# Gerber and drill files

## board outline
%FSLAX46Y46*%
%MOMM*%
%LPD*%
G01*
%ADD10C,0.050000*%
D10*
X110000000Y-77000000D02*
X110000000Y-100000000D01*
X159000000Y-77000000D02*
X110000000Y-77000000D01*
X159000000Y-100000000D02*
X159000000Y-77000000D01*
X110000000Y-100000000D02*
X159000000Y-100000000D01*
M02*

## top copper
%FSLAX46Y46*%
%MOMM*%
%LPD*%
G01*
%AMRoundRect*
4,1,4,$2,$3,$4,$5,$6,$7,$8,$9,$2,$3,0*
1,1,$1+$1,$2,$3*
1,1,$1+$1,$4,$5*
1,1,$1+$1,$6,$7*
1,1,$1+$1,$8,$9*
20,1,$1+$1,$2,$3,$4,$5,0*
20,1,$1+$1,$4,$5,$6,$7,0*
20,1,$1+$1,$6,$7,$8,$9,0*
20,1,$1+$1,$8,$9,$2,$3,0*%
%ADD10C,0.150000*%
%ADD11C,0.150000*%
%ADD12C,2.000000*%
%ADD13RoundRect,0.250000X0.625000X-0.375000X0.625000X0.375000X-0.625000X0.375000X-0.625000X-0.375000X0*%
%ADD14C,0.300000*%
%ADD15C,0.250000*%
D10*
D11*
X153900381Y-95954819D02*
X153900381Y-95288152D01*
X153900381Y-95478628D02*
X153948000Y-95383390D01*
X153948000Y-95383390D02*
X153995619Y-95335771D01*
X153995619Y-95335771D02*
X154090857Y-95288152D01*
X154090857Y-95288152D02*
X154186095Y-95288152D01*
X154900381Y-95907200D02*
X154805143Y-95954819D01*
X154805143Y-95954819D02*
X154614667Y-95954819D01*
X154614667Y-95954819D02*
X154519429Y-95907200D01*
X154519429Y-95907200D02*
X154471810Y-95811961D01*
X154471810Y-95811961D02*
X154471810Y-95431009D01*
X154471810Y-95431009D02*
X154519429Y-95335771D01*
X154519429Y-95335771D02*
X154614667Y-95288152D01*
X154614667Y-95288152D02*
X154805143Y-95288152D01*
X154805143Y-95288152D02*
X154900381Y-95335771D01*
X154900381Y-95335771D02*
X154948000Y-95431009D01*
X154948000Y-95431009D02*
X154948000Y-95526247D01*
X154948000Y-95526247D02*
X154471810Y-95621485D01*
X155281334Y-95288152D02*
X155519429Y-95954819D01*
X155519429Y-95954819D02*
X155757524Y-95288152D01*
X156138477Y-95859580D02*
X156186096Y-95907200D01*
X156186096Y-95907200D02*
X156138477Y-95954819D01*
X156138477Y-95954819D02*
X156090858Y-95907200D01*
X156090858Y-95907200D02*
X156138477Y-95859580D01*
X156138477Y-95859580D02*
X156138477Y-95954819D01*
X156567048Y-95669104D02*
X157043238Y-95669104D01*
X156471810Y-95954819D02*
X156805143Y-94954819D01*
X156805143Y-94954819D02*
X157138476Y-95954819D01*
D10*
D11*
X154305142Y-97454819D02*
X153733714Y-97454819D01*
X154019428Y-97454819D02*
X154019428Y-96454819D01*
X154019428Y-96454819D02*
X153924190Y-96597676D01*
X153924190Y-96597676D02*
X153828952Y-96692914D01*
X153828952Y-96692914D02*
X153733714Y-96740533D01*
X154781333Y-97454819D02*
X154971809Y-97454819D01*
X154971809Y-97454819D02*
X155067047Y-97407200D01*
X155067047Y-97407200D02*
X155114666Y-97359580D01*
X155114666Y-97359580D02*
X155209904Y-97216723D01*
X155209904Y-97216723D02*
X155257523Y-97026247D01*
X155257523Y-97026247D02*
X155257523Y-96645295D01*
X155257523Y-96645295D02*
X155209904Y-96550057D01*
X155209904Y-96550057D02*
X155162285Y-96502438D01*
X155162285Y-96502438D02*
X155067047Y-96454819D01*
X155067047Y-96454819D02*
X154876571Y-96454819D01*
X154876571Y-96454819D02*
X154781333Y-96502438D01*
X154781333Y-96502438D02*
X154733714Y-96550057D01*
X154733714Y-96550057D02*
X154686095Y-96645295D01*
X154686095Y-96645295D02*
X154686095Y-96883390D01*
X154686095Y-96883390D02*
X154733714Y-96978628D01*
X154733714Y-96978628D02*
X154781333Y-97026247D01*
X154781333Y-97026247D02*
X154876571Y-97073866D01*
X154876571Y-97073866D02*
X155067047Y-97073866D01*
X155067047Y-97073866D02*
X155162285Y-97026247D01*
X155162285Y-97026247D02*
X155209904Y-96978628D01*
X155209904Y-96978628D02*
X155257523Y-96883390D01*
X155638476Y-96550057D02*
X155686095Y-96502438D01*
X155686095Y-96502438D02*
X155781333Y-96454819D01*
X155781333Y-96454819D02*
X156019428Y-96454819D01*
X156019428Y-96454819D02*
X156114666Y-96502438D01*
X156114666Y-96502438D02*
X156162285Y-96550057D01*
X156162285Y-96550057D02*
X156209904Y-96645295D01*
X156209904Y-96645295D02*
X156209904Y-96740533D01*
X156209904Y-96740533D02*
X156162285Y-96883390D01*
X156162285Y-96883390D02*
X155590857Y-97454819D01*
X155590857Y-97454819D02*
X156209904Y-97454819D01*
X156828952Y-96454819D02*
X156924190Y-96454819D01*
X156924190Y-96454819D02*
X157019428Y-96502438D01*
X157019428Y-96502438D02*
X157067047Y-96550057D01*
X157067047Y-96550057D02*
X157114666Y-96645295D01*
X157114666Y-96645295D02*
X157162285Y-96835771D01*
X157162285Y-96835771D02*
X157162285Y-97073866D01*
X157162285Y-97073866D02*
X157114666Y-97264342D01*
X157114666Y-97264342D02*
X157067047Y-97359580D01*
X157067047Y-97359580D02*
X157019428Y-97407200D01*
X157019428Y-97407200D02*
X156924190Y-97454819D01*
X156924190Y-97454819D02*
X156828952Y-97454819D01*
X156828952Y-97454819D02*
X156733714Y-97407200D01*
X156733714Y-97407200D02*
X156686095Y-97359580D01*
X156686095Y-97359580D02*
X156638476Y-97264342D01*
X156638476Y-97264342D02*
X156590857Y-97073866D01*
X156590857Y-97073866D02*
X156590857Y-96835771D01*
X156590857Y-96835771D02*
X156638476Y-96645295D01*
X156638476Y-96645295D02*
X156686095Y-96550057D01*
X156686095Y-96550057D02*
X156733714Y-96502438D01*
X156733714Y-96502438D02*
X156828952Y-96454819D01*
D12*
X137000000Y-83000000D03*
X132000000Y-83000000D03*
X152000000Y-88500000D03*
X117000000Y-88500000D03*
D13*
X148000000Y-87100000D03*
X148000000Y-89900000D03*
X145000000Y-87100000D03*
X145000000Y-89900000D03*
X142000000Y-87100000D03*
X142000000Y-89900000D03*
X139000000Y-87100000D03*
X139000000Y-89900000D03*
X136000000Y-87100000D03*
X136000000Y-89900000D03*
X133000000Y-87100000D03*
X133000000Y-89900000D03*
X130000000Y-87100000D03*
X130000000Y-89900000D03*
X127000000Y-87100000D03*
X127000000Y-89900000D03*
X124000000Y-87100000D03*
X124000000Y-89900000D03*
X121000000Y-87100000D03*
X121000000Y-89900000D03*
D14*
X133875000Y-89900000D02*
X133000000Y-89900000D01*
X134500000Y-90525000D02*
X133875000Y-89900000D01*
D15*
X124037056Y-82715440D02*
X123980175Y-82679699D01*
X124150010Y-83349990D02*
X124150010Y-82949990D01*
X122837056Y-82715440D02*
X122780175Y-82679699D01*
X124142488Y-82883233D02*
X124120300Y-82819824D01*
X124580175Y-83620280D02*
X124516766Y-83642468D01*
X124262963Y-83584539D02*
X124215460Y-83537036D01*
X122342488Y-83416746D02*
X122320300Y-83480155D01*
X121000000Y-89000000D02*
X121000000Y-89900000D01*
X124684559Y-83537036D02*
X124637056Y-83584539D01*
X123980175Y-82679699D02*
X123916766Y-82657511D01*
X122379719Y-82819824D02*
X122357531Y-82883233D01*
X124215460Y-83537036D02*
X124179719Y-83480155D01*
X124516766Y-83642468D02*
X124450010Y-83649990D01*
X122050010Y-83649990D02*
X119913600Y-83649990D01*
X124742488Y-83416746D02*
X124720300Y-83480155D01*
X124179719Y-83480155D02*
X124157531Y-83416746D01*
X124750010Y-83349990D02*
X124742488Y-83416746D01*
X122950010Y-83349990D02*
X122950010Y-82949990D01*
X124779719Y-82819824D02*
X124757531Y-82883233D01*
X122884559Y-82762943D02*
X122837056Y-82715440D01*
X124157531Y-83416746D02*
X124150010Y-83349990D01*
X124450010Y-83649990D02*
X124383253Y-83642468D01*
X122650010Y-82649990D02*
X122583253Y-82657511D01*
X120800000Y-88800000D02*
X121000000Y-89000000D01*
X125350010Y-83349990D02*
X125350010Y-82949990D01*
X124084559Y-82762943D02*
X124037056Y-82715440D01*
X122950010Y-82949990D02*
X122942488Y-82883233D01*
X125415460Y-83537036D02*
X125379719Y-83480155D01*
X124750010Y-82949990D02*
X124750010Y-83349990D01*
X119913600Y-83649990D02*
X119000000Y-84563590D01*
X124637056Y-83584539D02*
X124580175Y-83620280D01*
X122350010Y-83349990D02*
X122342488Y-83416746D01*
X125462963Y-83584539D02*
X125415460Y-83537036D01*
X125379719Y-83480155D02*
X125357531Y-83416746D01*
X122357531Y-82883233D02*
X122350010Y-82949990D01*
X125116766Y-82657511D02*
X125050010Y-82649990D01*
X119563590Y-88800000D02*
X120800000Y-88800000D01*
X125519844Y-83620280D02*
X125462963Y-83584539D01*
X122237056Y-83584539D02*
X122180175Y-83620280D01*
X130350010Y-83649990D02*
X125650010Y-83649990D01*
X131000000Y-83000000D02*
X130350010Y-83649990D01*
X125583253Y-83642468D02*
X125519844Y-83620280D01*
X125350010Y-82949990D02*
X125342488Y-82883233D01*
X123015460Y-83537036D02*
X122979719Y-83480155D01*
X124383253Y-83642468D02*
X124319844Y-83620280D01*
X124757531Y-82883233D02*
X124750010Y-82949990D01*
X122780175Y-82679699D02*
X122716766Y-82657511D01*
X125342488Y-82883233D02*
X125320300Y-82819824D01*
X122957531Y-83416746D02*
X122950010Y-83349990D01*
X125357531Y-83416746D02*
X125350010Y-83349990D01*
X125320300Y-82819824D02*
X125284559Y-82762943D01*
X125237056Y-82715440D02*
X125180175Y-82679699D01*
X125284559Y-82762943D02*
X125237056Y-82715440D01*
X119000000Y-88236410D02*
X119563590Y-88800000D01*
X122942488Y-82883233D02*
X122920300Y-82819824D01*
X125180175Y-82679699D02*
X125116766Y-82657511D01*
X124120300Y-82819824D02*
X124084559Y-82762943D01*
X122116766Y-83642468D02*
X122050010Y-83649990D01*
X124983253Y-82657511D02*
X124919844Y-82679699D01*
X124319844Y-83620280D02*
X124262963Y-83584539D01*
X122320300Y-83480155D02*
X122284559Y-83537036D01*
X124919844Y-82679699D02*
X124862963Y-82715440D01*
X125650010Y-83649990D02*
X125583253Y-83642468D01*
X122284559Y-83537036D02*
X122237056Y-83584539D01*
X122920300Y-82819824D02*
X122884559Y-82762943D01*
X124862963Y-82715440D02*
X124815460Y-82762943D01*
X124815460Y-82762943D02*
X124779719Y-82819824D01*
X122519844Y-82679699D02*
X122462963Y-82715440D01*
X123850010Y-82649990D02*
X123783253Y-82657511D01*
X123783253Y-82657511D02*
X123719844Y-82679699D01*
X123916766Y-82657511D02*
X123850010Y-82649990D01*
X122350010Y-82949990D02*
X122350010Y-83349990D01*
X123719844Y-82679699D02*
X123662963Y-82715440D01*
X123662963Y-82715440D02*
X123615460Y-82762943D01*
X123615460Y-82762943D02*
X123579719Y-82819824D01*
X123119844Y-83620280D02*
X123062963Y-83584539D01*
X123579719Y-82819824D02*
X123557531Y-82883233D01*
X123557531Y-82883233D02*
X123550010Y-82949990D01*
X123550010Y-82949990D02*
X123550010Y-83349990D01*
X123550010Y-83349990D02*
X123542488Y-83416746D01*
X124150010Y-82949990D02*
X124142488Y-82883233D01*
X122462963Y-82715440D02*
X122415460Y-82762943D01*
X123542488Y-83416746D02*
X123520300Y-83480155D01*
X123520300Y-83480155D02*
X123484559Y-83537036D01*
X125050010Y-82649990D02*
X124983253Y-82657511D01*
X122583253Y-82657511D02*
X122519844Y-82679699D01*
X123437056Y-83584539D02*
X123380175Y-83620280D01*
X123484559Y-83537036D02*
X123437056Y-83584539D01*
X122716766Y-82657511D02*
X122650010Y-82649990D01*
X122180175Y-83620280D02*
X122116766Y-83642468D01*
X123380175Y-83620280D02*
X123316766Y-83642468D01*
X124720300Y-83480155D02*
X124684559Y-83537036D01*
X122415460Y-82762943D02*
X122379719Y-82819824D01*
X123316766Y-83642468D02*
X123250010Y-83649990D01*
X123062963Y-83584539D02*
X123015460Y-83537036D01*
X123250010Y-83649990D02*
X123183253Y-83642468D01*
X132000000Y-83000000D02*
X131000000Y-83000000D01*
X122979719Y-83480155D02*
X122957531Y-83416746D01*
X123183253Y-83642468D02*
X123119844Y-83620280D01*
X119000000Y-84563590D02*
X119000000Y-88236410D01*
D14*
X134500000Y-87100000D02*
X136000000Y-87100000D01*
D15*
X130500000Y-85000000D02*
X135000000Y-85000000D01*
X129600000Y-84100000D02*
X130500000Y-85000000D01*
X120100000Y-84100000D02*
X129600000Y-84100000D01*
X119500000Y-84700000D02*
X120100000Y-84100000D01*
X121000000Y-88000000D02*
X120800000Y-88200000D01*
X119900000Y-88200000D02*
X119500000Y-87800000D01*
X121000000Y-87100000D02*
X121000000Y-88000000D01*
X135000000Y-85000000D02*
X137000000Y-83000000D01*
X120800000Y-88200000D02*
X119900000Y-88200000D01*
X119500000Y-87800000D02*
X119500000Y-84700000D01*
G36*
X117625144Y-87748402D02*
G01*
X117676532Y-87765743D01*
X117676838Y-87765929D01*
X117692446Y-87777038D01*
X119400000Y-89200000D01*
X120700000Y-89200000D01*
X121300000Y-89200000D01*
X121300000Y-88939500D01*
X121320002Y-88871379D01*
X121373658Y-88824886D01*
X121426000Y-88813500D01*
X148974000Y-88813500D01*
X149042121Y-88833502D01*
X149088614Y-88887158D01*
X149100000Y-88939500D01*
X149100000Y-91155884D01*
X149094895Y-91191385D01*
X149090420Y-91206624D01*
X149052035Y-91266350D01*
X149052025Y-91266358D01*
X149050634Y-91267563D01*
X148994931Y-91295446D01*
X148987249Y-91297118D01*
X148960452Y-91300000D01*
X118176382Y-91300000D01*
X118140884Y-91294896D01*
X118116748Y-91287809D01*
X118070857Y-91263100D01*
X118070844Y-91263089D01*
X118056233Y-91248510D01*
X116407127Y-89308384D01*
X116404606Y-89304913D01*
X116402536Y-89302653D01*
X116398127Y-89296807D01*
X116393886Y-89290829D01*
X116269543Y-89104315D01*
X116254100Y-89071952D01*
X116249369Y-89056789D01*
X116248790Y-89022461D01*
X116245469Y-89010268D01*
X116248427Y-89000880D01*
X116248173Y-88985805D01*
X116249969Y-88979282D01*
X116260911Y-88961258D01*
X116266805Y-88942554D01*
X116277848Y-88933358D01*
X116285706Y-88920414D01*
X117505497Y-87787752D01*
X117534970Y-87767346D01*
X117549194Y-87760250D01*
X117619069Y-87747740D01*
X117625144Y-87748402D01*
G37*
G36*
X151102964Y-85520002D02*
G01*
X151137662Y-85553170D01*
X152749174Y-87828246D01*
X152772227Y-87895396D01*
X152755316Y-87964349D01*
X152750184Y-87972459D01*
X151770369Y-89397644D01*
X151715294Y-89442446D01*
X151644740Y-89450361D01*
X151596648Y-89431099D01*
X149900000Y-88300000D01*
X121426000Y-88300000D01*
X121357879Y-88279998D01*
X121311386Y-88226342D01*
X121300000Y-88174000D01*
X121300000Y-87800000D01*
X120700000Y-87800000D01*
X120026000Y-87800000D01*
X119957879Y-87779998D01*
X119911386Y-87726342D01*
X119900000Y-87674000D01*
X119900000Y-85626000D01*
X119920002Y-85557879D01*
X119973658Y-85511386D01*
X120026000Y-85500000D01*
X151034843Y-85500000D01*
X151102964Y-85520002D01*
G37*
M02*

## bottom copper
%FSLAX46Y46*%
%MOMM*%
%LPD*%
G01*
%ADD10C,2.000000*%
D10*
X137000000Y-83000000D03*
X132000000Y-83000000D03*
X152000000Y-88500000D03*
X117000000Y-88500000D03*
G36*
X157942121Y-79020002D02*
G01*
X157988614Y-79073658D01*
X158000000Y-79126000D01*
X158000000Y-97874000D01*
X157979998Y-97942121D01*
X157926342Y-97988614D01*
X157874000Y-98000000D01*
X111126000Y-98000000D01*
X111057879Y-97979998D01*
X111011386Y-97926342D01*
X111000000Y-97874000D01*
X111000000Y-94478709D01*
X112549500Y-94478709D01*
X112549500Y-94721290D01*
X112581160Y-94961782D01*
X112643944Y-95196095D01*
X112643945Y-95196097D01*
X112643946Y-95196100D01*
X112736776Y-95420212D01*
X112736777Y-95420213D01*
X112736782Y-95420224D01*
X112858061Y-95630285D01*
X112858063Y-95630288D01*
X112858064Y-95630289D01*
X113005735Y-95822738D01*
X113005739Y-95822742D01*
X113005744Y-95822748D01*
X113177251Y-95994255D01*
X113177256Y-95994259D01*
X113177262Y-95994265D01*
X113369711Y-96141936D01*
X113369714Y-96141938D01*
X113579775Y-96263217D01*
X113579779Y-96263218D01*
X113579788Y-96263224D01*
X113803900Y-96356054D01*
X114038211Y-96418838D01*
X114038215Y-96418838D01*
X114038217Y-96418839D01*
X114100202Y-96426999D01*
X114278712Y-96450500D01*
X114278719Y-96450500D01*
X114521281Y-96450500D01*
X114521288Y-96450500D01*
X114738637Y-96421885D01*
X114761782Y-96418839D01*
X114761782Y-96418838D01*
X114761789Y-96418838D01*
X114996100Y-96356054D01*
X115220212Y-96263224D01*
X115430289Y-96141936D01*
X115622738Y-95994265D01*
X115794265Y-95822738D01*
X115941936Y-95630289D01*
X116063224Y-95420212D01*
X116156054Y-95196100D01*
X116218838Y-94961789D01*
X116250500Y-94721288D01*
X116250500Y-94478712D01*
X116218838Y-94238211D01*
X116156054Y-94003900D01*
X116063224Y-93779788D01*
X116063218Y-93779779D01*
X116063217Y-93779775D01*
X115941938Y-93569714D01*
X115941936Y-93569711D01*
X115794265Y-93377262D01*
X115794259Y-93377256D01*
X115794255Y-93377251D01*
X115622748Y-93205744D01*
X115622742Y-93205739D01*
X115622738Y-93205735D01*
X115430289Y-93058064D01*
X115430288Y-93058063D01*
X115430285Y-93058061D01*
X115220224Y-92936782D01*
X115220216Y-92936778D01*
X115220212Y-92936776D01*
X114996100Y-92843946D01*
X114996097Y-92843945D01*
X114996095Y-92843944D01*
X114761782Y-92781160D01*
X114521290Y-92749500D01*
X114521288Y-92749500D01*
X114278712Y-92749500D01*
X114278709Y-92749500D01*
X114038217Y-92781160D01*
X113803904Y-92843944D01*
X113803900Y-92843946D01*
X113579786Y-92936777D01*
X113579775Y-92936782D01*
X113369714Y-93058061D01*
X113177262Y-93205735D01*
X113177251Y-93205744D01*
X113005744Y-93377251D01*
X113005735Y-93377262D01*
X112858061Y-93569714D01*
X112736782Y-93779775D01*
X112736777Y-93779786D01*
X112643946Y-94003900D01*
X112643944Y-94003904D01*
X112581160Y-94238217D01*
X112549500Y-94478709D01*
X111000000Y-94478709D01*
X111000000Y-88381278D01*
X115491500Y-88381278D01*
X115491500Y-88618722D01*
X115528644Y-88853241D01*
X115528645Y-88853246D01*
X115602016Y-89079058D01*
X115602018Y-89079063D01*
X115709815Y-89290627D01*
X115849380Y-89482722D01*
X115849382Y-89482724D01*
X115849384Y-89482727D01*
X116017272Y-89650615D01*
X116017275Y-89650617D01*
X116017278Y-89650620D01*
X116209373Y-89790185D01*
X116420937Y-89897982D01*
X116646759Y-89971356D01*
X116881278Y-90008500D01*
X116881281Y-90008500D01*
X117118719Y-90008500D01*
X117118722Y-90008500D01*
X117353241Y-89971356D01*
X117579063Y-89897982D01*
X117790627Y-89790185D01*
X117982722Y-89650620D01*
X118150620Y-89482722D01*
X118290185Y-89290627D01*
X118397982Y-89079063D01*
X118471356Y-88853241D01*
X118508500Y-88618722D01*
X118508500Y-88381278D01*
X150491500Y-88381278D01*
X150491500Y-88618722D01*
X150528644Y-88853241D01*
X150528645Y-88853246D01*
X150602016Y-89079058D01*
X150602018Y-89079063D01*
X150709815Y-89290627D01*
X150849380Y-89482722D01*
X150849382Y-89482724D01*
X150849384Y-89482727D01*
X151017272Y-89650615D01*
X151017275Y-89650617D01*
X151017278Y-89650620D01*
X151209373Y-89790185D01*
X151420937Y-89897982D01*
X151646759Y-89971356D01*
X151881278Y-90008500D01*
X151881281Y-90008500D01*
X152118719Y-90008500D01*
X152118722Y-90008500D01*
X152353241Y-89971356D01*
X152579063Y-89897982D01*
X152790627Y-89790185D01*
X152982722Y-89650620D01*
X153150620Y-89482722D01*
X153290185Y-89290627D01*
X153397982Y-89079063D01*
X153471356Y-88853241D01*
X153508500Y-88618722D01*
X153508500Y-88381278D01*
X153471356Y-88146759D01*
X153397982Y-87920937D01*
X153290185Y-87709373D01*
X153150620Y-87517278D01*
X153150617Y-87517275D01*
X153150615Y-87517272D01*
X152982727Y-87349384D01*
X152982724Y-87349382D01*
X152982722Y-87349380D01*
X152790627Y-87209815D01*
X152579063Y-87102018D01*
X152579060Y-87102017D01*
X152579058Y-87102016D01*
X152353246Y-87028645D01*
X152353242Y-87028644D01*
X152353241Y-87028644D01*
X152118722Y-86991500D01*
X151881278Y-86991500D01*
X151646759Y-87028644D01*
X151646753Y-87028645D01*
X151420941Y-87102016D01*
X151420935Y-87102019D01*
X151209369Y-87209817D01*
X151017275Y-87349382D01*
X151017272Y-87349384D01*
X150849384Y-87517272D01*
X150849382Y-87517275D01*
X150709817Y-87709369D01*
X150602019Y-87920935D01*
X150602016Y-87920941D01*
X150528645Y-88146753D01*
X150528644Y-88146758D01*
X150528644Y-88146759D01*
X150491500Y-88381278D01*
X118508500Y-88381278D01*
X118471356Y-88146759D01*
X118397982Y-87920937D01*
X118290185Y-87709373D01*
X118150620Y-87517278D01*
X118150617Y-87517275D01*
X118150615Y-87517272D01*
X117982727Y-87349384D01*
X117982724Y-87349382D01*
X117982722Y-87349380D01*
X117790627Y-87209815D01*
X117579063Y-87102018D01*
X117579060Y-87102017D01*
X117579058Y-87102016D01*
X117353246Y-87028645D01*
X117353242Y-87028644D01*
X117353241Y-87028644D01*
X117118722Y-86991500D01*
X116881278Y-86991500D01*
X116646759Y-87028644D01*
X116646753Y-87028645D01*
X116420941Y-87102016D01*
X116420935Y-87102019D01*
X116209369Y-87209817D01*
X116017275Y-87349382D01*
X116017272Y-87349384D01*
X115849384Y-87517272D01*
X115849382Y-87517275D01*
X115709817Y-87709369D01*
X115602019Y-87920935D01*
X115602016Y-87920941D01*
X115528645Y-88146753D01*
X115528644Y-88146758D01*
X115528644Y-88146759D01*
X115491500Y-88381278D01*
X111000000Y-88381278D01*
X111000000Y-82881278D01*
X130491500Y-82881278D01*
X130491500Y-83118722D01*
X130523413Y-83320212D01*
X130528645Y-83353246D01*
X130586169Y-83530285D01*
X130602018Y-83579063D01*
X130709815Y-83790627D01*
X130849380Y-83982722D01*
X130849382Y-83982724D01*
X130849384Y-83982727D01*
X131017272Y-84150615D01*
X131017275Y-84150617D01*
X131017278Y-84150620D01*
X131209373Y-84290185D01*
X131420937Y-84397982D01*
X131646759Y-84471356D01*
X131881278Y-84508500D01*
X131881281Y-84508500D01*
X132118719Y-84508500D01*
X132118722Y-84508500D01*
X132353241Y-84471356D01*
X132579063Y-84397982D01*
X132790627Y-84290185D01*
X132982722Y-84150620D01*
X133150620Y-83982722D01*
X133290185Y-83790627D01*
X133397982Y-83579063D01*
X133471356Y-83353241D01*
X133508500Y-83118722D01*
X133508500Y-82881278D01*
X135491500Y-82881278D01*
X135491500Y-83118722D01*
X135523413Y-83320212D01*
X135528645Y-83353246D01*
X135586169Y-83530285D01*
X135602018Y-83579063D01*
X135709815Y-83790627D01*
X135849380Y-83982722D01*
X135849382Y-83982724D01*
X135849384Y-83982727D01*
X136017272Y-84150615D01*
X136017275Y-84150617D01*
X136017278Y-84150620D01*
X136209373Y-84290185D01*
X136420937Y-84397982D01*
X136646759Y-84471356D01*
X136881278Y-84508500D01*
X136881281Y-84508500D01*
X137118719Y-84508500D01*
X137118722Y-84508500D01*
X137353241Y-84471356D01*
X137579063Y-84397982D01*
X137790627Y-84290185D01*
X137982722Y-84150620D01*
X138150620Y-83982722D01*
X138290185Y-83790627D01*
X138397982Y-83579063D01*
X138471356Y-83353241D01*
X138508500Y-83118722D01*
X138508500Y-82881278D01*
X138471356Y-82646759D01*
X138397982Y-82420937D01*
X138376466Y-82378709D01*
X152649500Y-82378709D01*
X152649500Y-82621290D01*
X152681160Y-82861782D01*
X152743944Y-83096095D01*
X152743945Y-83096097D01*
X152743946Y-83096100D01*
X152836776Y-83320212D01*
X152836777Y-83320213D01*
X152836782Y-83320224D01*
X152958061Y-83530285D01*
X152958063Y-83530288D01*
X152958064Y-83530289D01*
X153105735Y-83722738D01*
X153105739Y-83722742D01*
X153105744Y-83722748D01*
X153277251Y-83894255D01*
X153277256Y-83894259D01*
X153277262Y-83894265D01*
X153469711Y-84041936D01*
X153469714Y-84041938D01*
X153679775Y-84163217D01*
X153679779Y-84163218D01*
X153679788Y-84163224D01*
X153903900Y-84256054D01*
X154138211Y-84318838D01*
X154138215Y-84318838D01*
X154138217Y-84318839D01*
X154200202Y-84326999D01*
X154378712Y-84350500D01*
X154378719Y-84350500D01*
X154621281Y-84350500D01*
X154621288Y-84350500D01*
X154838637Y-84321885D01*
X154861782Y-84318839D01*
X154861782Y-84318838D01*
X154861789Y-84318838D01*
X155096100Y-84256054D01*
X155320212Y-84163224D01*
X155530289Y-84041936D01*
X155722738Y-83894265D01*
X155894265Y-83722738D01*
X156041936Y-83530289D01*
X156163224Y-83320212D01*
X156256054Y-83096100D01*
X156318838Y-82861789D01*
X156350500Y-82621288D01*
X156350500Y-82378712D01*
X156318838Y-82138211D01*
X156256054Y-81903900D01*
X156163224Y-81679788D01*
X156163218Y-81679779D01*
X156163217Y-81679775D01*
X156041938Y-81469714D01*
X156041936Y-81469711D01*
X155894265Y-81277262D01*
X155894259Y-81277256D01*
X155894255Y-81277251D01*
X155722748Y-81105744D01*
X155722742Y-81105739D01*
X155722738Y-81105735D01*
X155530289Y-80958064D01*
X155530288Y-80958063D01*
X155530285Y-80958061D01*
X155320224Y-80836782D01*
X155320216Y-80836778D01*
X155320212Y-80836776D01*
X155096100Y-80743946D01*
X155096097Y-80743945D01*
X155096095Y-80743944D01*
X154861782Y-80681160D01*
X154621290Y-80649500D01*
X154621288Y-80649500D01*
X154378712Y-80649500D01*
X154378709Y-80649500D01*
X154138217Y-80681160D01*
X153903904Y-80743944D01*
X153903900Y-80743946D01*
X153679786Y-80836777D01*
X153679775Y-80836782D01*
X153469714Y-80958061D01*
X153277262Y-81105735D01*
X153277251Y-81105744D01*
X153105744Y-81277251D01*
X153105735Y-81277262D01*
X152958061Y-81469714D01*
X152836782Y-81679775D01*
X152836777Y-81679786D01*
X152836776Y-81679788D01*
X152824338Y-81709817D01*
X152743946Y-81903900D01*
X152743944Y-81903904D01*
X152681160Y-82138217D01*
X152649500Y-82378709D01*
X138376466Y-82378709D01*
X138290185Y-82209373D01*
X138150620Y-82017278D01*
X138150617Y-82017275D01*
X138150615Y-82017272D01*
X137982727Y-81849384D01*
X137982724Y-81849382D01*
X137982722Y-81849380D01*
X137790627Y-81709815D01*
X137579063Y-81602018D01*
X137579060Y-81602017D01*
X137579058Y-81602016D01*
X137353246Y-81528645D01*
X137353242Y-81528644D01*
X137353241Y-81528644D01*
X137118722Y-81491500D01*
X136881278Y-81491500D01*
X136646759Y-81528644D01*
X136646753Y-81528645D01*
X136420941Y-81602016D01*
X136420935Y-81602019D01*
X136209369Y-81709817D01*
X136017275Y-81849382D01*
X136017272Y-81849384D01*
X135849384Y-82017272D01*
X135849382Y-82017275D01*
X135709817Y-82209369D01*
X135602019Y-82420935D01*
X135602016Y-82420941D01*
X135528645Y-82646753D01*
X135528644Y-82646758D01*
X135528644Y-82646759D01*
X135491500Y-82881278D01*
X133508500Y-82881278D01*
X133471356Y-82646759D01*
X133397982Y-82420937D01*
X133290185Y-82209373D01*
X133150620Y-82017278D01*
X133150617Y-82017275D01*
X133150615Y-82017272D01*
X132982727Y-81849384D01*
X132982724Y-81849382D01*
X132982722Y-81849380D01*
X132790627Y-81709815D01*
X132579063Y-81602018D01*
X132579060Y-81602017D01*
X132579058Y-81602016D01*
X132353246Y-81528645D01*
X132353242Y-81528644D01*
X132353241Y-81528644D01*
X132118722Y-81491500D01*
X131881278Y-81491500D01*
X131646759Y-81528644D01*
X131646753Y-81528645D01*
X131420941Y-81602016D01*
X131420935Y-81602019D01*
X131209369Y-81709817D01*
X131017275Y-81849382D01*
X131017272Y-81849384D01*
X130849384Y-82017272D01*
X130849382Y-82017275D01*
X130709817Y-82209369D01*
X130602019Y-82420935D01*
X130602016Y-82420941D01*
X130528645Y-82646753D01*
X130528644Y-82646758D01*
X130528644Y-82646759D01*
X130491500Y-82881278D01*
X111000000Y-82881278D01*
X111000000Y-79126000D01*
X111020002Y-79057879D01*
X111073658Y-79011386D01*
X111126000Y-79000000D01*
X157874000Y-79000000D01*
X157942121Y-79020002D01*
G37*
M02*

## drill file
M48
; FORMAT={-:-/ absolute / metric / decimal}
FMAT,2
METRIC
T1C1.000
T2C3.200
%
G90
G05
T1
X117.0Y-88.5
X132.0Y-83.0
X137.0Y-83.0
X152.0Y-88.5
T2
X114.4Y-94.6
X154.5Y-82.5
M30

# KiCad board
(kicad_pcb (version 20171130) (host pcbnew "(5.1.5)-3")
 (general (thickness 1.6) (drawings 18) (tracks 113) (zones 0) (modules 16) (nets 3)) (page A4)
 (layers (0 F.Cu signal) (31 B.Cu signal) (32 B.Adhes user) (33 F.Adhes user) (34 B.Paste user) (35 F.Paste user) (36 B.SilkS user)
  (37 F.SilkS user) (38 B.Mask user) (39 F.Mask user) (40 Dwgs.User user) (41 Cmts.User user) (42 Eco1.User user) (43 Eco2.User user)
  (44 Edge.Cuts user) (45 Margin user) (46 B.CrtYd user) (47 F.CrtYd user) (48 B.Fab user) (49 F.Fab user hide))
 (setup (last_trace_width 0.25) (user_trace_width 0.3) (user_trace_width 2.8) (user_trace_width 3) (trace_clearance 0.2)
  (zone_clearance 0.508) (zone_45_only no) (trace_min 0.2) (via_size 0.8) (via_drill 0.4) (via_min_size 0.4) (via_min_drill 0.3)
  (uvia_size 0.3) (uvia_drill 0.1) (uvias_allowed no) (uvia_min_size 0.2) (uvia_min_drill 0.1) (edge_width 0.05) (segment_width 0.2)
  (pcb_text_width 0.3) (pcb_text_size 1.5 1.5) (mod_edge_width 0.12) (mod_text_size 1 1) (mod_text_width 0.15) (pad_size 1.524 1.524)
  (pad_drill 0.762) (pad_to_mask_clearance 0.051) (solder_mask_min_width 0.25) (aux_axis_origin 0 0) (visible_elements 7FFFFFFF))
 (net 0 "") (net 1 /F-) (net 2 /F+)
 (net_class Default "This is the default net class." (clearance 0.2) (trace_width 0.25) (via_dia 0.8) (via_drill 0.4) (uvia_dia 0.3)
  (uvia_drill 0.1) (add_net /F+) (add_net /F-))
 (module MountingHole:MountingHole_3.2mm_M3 (layer F.Cu) (at 154.5 82.5)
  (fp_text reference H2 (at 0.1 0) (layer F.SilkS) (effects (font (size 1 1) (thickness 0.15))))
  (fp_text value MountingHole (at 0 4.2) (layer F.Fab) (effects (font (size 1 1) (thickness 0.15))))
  (pad 1 np_thru_hole circle (at 0 0) (size 3.2 3.2) (drill 3.2) (layers *.Cu *.Mask)))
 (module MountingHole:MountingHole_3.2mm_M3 (layer F.Cu) (at 114.4 94.6)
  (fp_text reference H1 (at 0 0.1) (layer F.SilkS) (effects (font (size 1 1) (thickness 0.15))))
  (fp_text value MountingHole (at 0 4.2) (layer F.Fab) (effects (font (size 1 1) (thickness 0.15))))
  (pad 1 np_thru_hole circle (at 0 0) (size 3.2 3.2) (drill 3.2) (layers *.Cu *.Mask)))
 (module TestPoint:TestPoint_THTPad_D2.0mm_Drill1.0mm (layer F.Cu) (at 137 83)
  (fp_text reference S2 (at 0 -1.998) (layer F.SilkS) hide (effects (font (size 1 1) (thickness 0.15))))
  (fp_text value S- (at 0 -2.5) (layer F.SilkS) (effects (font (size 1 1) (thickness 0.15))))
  (pad 1 thru_hole circle (at 0 0) (size 2 2) (drill 1) (layers *.Cu *.Mask) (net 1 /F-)))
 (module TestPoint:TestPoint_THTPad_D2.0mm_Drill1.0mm (layer F.Cu) (at 132 83)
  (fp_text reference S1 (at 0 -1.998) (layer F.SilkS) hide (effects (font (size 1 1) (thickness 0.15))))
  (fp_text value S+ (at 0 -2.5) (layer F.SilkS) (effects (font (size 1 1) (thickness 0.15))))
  (pad 1 thru_hole circle (at 0 0) (size 2 2) (drill 1) (layers *.Cu *.Mask) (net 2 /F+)))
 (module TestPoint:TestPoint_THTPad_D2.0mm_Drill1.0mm (layer F.Cu) (at 152 88.5)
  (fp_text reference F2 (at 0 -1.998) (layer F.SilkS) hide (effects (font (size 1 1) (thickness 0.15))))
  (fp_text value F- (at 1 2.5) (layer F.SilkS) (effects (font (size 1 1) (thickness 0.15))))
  (pad 1 thru_hole circle (at 0 0) (size 2 2) (drill 1) (layers *.Cu *.Mask) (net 1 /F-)))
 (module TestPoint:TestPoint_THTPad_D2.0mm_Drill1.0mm (layer F.Cu) (at 117 88.5)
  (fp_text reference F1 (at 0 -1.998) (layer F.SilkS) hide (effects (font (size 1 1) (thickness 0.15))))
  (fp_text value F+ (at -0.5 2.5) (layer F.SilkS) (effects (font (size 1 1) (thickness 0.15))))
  (pad 1 thru_hole circle (at 0 0) (size 2 2) (drill 1) (layers *.Cu *.Mask) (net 2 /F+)))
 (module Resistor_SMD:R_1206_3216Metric (layer F.Cu) (at 148 88.5 90)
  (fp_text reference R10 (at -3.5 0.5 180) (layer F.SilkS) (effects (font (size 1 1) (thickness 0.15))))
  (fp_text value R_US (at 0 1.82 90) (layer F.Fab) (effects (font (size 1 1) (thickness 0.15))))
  (pad 2 smd roundrect (at 1.4 0 90) (size 1.25 1.75) (layers F.Cu F.Paste F.Mask) (roundrect_rratio 0.2) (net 1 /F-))
  (pad 1 smd roundrect (at -1.4 0 90) (size 1.25 1.75) (layers F.Cu F.Paste F.Mask) (roundrect_rratio 0.2) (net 2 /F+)))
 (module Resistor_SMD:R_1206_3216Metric (layer F.Cu) (at 145 88.5 90)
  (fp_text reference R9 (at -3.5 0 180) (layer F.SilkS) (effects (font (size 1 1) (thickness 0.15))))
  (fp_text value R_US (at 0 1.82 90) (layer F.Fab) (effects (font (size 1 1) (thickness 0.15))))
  (pad 2 smd roundrect (at 1.4 0 90) (size 1.25 1.75) (layers F.Cu F.Paste F.Mask) (roundrect_rratio 0.2) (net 1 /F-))
  (pad 1 smd roundrect (at -1.4 0 90) (size 1.25 1.75) (layers F.Cu F.Paste F.Mask) (roundrect_rratio 0.2) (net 2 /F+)))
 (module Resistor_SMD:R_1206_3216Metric (layer F.Cu) (at 142 88.5 90)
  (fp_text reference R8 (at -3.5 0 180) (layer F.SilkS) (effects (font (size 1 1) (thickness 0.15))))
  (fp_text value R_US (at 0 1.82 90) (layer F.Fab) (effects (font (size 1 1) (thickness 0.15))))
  (pad 2 smd roundrect (at 1.4 0 90) (size 1.25 1.75) (layers F.Cu F.Paste F.Mask) (roundrect_rratio 0.2) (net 1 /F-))
  (pad 1 smd roundrect (at -1.4 0 90) (size 1.25 1.75) (layers F.Cu F.Paste F.Mask) (roundrect_rratio 0.2) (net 2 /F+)))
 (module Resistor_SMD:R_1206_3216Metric (layer F.Cu) (at 139 88.5 90)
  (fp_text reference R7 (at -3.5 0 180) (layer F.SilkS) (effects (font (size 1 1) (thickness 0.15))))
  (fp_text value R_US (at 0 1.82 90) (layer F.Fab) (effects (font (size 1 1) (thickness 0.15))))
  (pad 2 smd roundrect (at 1.4 0 90) (size 1.25 1.75) (layers F.Cu F.Paste F.Mask) (roundrect_rratio 0.2) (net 1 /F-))
  (pad 1 smd roundrect (at -1.4 0 90) (size 1.25 1.75) (layers F.Cu F.Paste F.Mask) (roundrect_rratio 0.2) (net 2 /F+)))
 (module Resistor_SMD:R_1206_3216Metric (layer F.Cu) (at 136 88.5 90)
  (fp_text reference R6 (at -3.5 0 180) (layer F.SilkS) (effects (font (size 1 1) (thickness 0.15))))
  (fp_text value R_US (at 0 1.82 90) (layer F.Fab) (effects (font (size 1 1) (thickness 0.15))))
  (pad 2 smd roundrect (at 1.4 0 90) (size 1.25 1.75) (layers F.Cu F.Paste F.Mask) (roundrect_rratio 0.2) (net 1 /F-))
  (pad 1 smd roundrect (at -1.4 0 90) (size 1.25 1.75) (layers F.Cu F.Paste F.Mask) (roundrect_rratio 0.2) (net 2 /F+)))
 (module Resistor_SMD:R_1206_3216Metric (layer F.Cu) (at 133 88.5 90)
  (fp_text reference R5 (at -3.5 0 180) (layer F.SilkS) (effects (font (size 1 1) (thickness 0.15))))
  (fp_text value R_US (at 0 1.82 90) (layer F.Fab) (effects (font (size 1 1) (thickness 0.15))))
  (pad 2 smd roundrect (at 1.4 0 90) (size 1.25 1.75) (layers F.Cu F.Paste F.Mask) (roundrect_rratio 0.2) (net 1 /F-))
  (pad 1 smd roundrect (at -1.4 0 90) (size 1.25 1.75) (layers F.Cu F.Paste F.Mask) (roundrect_rratio 0.2) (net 2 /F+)))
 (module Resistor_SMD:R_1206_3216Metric (layer F.Cu) (at 130 88.5 90)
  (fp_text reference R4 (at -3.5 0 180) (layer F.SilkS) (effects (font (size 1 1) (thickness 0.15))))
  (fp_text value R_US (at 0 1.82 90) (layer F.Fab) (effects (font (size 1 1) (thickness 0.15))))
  (pad 2 smd roundrect (at 1.4 0 90) (size 1.25 1.75) (layers F.Cu F.Paste F.Mask) (roundrect_rratio 0.2) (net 1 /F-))
  (pad 1 smd roundrect (at -1.4 0 90) (size 1.25 1.75) (layers F.Cu F.Paste F.Mask) (roundrect_rratio 0.2) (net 2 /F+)))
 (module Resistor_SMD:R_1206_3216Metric (layer F.Cu) (at 127 88.5 90)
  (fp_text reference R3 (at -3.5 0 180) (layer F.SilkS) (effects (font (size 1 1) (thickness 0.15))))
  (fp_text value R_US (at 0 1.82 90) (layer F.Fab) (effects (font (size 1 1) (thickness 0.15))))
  (pad 2 smd roundrect (at 1.4 0 90) (size 1.25 1.75) (layers F.Cu F.Paste F.Mask) (roundrect_rratio 0.2) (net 1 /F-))
  (pad 1 smd roundrect (at -1.4 0 90) (size 1.25 1.75) (layers F.Cu F.Paste F.Mask) (roundrect_rratio 0.2) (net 2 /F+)))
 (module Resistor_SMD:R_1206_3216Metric (layer F.Cu) (at 124 88.5 90)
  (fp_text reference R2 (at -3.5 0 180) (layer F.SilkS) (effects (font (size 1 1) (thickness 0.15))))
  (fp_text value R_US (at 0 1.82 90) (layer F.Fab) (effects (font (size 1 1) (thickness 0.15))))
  (pad 2 smd roundrect (at 1.4 0 90) (size 1.25 1.75) (layers F.Cu F.Paste F.Mask) (roundrect_rratio 0.2) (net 1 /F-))
  (pad 1 smd roundrect (at -1.4 0 90) (size 1.25 1.75) (layers F.Cu F.Paste F.Mask) (roundrect_rratio 0.2) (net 2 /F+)))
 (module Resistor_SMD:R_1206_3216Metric (layer F.Cu) (at 121 88.5 90)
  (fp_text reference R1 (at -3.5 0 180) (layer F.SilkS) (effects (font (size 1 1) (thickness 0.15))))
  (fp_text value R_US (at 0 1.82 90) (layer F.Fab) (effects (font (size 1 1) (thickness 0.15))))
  (pad 2 smd roundrect (at 1.4 0 90) (size 1.25 1.75) (layers F.Cu F.Paste F.Mask) (roundrect_rratio 0.2) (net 1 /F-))
  (pad 1 smd roundrect (at -1.4 0 90) (size 1.25 1.75) (layers F.Cu F.Paste F.Mask) (roundrect_rratio 0.2) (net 2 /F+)))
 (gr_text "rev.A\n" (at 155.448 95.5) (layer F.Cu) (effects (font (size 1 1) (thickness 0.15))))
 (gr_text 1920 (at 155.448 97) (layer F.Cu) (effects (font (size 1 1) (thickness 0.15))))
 (gr_line (start 110 77) (end 110 100) (layer Edge.Cuts) (width 0.05))
 (gr_line (start 159 77) (end 110 77) (layer Edge.Cuts) (width 0.05))
 (gr_line (start 159 100) (end 159 77) (layer Edge.Cuts) (width 0.05))
 (gr_line (start 110 100) (end 159 100) (layer Edge.Cuts) (width 0.05))
 (segment (start 133.875 89.9) (end 133 89.9) (width 0.3) (layer F.Cu) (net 2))
 (segment (start 134.5 90.525) (end 133.875 89.9) (width 0.3) (layer F.Cu) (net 2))
 (segment (start 124.037056 82.71544) (end 123.980175 82.679699) (width 0.25) (layer F.Cu) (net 2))
 (segment (start 124.15001 83.34999) (end 124.15001 82.94999) (width 0.25) (layer F.Cu) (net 2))
 (segment (start 122.837056 82.71544) (end 122.780175 82.679699) (width 0.25) (layer F.Cu) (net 2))
 (segment (start 124.142488 82.883233) (end 124.1203 82.819824) (width 0.25) (layer F.Cu) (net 2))
 (segment (start 124.580175 83.62028) (end 124.516766 83.642468) (width 0.25) (layer F.Cu) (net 2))
 (segment (start 124.262963 83.584539) (end 124.21546 83.537036) (width 0.25) (layer F.Cu) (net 2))
 (segment (start 122.342488 83.416746) (end 122.3203 83.480155) (width 0.25) (layer F.Cu) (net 2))
 (segment (start 121 89) (end 121 89.9) (width 0.25) (layer F.Cu) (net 2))
 (segment (start 124.684559 83.537036) (end 124.637056 83.584539) (width 0.25) (layer F.Cu) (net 2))
 (segment (start 123.980175 82.679699) (end 123.916766 82.657511) (width 0.25) (layer F.Cu) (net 2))
 (segment (start 122.379719 82.819824) (end 122.357531 82.883233) (width 0.25) (layer F.Cu) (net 2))
 (segment (start 124.21546 83.537036) (end 124.179719 83.480155) (width 0.25) (layer F.Cu) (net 2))
 (segment (start 124.516766 83.642468) (end 124.45001 83.64999) (width 0.25) (layer F.Cu) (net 2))
 (segment (start 122.05001 83.64999) (end 119.9136 83.64999) (width 0.25) (layer F.Cu) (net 2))
 (segment (start 124.742488 83.416746) (end 124.7203 83.480155) (width 0.25) (layer F.Cu) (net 2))
 (segment (start 124.179719 83.480155) (end 124.157531 83.416746) (width 0.25) (layer F.Cu) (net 2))
 (segment (start 124.75001 83.34999) (end 124.742488 83.416746) (width 0.25) (layer F.Cu) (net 2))
 (segment (start 122.95001 83.34999) (end 122.95001 82.94999) (width 0.25) (layer F.Cu) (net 2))
 (segment (start 124.779719 82.819824) (end 124.757531 82.883233) (width 0.25) (layer F.Cu) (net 2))
 (segment (start 122.884559 82.762943) (end 122.837056 82.71544) (width 0.25) (layer F.Cu) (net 2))
 (segment (start 124.157531 83.416746) (end 124.15001 83.34999) (width 0.25) (layer F.Cu) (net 2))
 (segment (start 124.45001 83.64999) (end 124.383253 83.642468) (width 0.25) (layer F.Cu) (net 2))
 (segment (start 122.65001 82.64999) (end 122.583253 82.657511) (width 0.25) (layer F.Cu) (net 2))
 (segment (start 120.8 88.8) (end 121 89) (width 0.25) (layer F.Cu) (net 2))
 (segment (start 125.35001 83.34999) (end 125.35001 82.94999) (width 0.25) (layer F.Cu) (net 2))
 (segment (start 124.084559 82.762943) (end 124.037056 82.71544) (width 0.25) (layer F.Cu) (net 2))
 (segment (start 122.95001 82.94999) (end 122.942488 82.883233) (width 0.25) (layer F.Cu) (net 2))
 (segment (start 125.41546 83.537036) (end 125.379719 83.480155) (width 0.25) (layer F.Cu) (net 2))
 (segment (start 124.75001 82.94999) (end 124.75001 83.34999) (width 0.25) (layer F.Cu) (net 2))
 (segment (start 119.9136 83.64999) (end 119 84.56359) (width 0.25) (layer F.Cu) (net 2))
 (segment (start 124.637056 83.584539) (end 124.580175 83.62028) (width 0.25) (layer F.Cu) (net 2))
 (segment (start 122.35001 83.34999) (end 122.342488 83.416746) (width 0.25) (layer F.Cu) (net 2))
 (segment (start 125.462963 83.584539) (end 125.41546 83.537036) (width 0.25) (layer F.Cu) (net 2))
 (segment (start 125.379719 83.480155) (end 125.357531 83.416746) (width 0.25) (layer F.Cu) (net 2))
 (segment (start 122.357531 82.883233) (end 122.35001 82.94999) (width 0.25) (layer F.Cu) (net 2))
 (segment (start 125.116766 82.657511) (end 125.05001 82.64999) (width 0.25) (layer F.Cu) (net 2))
 (segment (start 119.56359 88.8) (end 120.8 88.8) (width 0.25) (layer F.Cu) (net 2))
 (segment (start 125.519844 83.62028) (end 125.462963 83.584539) (width 0.25) (layer F.Cu) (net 2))
 (segment (start 122.237056 83.584539) (end 122.180175 83.62028) (width 0.25) (layer F.Cu) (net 2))
 (segment (start 130.35001 83.64999) (end 125.65001 83.64999) (width 0.25) (layer F.Cu) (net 2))
 (segment (start 131 83) (end 130.35001 83.64999) (width 0.25) (layer F.Cu) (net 2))
 (segment (start 125.583253 83.642468) (end 125.519844 83.62028) (width 0.25) (layer F.Cu) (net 2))
 (segment (start 125.35001 82.94999) (end 125.342488 82.883233) (width 0.25) (layer F.Cu) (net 2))
 (segment (start 123.01546 83.537036) (end 122.979719 83.480155) (width 0.25) (layer F.Cu) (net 2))
 (segment (start 124.383253 83.642468) (end 124.319844 83.62028) (width 0.25) (layer F.Cu) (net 2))
 (segment (start 124.757531 82.883233) (end 124.75001 82.94999) (width 0.25) (layer F.Cu) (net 2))
 (segment (start 122.780175 82.679699) (end 122.716766 82.657511) (width 0.25) (layer F.Cu) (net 2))
 (segment (start 125.342488 82.883233) (end 125.3203 82.819824) (width 0.25) (layer F.Cu) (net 2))
 (segment (start 122.957531 83.416746) (end 122.95001 83.34999) (width 0.25) (layer F.Cu) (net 2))
 (segment (start 125.357531 83.416746) (end 125.35001 83.34999) (width 0.25) (layer F.Cu) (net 2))
 (segment (start 125.3203 82.819824) (end 125.284559 82.762943) (width 0.25) (layer F.Cu) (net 2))
 (segment (start 125.237056 82.71544) (end 125.180175 82.679699) (width 0.25) (layer F.Cu) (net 2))
 (segment (start 125.284559 82.762943) (end 125.237056 82.71544) (width 0.25) (layer F.Cu) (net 2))
 (segment (start 119 88.23641) (end 119.56359 88.8) (width 0.25) (layer F.Cu) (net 2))
 (segment (start 122.942488 82.883233) (end 122.9203 82.819824) (width 0.25) (layer F.Cu) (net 2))
 (segment (start 125.180175 82.679699) (end 125.116766 82.657511) (width 0.25) (layer F.Cu) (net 2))
 (segment (start 124.1203 82.819824) (end 124.084559 82.762943) (width 0.25) (layer F.Cu) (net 2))
 (segment (start 122.116766 83.642468) (end 122.05001 83.64999) (width 0.25) (layer F.Cu) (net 2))
 (segment (start 124.983253 82.657511) (end 124.919844 82.679699) (width 0.25) (layer F.Cu) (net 2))
 (segment (start 124.319844 83.62028) (end 124.262963 83.584539) (width 0.25) (layer F.Cu) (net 2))
 (segment (start 122.3203 83.480155) (end 122.284559 83.537036) (width 0.25) (layer F.Cu) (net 2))
 (segment (start 124.919844 82.679699) (end 124.862963 82.71544) (width 0.25) (layer F.Cu) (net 2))
 (segment (start 125.65001 83.64999) (end 125.583253 83.642468) (width 0.25) (layer F.Cu) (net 2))
 (segment (start 122.284559 83.537036) (end 122.237056 83.584539) (width 0.25) (layer F.Cu) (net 2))
 (segment (start 122.9203 82.819824) (end 122.884559 82.762943) (width 0.25) (layer F.Cu) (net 2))
 (segment (start 124.862963 82.71544) (end 124.81546 82.762943) (width 0.25) (layer F.Cu) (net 2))
 (segment (start 124.81546 82.762943) (end 124.779719 82.819824) (width 0.25) (layer F.Cu) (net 2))
 (segment (start 122.519844 82.679699) (end 122.462963 82.71544) (width 0.25) (layer F.Cu) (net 2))
 (segment (start 123.85001 82.64999) (end 123.783253 82.657511) (width 0.25) (layer F.Cu) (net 2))
 (segment (start 123.783253 82.657511) (end 123.719844 82.679699) (width 0.25) (layer F.Cu) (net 2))
 (segment (start 123.916766 82.657511) (end 123.85001 82.64999) (width 0.25) (layer F.Cu) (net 2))
 (segment (start 122.35001 82.94999) (end 122.35001 83.34999) (width 0.25) (layer F.Cu) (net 2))
 (segment (start 123.719844 82.679699) (end 123.662963 82.71544) (width 0.25) (layer F.Cu) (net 2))
 (segment (start 123.662963 82.71544) (end 123.61546 82.762943) (width 0.25) (layer F.Cu) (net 2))
 (segment (start 123.61546 82.762943) (end 123.579719 82.819824) (width 0.25) (layer F.Cu) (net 2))
 (segment (start 123.119844 83.62028) (end 123.062963 83.584539) (width 0.25) (layer F.Cu) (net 2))
 (segment (start 123.579719 82.819824) (end 123.557531 82.883233) (width 0.25) (layer F.Cu) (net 2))
 (segment (start 123.557531 82.883233) (end 123.55001 82.94999) (width 0.25) (layer F.Cu) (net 2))
 (segment (start 123.55001 82.94999) (end 123.55001 83.34999) (width 0.25) (layer F.Cu) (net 2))
 (segment (start 123.55001 83.34999) (end 123.542488 83.416746) (width 0.25) (layer F.Cu) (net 2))
 (segment (start 124.15001 82.94999) (end 124.142488 82.883233) (width 0.25) (layer F.Cu) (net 2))
 (segment (start 122.462963 82.71544) (end 122.41546 82.762943) (width 0.25) (layer F.Cu) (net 2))
 (segment (start 123.542488 83.416746) (end 123.5203 83.480155) (width 0.25) (layer F.Cu) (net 2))
 (segment (start 123.5203 83.480155) (end 123.484559 83.537036) (width 0.25) (layer F.Cu) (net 2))
 (segment (start 125.05001 82.64999) (end 124.983253 82.657511) (width 0.25) (layer F.Cu) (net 2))
 (segment (start 122.583253 82.657511) (end 122.519844 82.679699) (width 0.25) (layer F.Cu) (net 2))
 (segment (start 123.437056 83.584539) (end 123.380175 83.62028) (width 0.25) (layer F.Cu) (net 2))
 (segment (start 123.484559 83.537036) (end 123.437056 83.584539) (width 0.25) (layer F.Cu) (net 2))
 (segment (start 122.716766 82.657511) (end 122.65001 82.64999) (width 0.25) (layer F.Cu) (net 2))
 (segment (start 122.180175 83.62028) (end 122.116766 83.642468) (width 0.25) (layer F.Cu) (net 2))
 (segment (start 123.380175 83.62028) (end 123.316766 83.642468) (width 0.25) (layer F.Cu) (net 2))
 (segment (start 124.7203 83.480155) (end 124.684559 83.537036) (width 0.25) (layer F.Cu) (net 2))
 (segment (start 122.41546 82.762943) (end 122.379719 82.819824) (width 0.25) (layer F.Cu) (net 2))
 (segment (start 123.316766 83.642468) (end 123.25001 83.64999) (width 0.25) (layer F.Cu) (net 2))
 (segment (start 123.062963 83.584539) (end 123.01546 83.537036) (width 0.25) (layer F.Cu) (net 2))
 (segment (start 123.25001 83.64999) (end 123.183253 83.642468) (width 0.25) (layer F.Cu) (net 2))
 (segment (start 132 83) (end 131 83) (width 0.25) (layer F.Cu) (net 2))
 (segment (start 122.979719 83.480155) (end 122.957531 83.416746) (width 0.25) (layer F.Cu) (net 2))
 (segment (start 123.183253 83.642468) (end 123.119844 83.62028) (width 0.25) (layer F.Cu) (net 2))
 (segment (start 119 84.56359) (end 119 88.23641) (width 0.25) (layer F.Cu) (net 2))
 (segment (start 134.5 87.1) (end 136 87.1) (width 0.3) (layer F.Cu) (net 1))
 (segment (start 130.5 85) (end 135 85) (width 0.25) (layer F.Cu) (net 1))
 (segment (start 129.6 84.1) (end 130.5 85) (width 0.25) (layer F.Cu) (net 1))
 (segment (start 120.1 84.1) (end 129.6 84.1) (width 0.25) (layer F.Cu) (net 1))
 (segment (start 119.5 84.7) (end 120.1 84.1) (width 0.25) (layer F.Cu) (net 1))
 (segment (start 121 88) (end 120.8 88.2) (width 0.25) (layer F.Cu) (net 1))
 (segment (start 119.9 88.2) (end 119.5 87.8) (width 0.25) (layer F.Cu) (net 1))
 (segment (start 121 87.1) (end 121 88) (width 0.25) (layer F.Cu) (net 1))
 (segment (start 135 85) (end 137 83) (width 0.25) (layer F.Cu) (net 1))
 (segment (start 120.8 88.2) (end 119.9 88.2) (width 0.25) (layer F.Cu) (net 1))
 (segment (start 119.5 87.8) (end 119.5 84.7) (width 0.25) (layer F.Cu) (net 1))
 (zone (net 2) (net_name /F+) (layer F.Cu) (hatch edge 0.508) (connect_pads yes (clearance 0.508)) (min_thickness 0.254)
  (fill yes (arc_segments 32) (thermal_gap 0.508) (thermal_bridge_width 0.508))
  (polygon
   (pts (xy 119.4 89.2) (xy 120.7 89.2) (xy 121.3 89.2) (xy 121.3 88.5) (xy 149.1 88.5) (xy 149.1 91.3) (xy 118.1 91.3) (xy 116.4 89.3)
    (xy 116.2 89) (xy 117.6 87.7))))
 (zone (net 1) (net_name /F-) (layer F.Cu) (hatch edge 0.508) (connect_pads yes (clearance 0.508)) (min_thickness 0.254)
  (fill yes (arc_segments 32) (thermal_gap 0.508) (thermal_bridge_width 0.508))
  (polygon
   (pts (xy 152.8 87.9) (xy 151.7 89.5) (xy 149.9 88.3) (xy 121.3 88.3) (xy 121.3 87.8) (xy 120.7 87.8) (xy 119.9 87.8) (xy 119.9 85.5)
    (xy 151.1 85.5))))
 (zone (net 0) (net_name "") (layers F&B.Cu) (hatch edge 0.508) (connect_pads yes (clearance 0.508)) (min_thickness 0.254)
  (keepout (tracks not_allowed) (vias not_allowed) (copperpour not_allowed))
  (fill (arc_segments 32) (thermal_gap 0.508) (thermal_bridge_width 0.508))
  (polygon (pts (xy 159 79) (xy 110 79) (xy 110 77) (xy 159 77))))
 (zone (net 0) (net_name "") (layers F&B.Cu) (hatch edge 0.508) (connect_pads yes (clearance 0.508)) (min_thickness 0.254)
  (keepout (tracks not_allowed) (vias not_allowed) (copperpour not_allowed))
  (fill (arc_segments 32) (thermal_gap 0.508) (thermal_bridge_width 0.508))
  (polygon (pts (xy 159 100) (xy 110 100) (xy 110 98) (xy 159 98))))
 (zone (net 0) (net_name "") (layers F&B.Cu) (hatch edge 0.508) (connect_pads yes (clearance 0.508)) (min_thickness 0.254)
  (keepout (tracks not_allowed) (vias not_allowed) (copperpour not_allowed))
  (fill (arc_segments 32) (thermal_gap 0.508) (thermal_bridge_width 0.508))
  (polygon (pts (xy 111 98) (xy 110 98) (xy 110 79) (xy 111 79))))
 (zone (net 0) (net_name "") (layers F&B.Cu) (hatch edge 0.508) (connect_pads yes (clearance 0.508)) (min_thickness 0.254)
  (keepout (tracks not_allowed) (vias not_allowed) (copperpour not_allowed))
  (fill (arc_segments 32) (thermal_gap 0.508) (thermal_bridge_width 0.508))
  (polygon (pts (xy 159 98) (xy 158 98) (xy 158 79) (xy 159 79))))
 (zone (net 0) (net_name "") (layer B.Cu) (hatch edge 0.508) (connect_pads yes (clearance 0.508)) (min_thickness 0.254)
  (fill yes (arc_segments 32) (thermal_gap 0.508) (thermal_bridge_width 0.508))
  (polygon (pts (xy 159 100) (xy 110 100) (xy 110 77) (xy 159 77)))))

